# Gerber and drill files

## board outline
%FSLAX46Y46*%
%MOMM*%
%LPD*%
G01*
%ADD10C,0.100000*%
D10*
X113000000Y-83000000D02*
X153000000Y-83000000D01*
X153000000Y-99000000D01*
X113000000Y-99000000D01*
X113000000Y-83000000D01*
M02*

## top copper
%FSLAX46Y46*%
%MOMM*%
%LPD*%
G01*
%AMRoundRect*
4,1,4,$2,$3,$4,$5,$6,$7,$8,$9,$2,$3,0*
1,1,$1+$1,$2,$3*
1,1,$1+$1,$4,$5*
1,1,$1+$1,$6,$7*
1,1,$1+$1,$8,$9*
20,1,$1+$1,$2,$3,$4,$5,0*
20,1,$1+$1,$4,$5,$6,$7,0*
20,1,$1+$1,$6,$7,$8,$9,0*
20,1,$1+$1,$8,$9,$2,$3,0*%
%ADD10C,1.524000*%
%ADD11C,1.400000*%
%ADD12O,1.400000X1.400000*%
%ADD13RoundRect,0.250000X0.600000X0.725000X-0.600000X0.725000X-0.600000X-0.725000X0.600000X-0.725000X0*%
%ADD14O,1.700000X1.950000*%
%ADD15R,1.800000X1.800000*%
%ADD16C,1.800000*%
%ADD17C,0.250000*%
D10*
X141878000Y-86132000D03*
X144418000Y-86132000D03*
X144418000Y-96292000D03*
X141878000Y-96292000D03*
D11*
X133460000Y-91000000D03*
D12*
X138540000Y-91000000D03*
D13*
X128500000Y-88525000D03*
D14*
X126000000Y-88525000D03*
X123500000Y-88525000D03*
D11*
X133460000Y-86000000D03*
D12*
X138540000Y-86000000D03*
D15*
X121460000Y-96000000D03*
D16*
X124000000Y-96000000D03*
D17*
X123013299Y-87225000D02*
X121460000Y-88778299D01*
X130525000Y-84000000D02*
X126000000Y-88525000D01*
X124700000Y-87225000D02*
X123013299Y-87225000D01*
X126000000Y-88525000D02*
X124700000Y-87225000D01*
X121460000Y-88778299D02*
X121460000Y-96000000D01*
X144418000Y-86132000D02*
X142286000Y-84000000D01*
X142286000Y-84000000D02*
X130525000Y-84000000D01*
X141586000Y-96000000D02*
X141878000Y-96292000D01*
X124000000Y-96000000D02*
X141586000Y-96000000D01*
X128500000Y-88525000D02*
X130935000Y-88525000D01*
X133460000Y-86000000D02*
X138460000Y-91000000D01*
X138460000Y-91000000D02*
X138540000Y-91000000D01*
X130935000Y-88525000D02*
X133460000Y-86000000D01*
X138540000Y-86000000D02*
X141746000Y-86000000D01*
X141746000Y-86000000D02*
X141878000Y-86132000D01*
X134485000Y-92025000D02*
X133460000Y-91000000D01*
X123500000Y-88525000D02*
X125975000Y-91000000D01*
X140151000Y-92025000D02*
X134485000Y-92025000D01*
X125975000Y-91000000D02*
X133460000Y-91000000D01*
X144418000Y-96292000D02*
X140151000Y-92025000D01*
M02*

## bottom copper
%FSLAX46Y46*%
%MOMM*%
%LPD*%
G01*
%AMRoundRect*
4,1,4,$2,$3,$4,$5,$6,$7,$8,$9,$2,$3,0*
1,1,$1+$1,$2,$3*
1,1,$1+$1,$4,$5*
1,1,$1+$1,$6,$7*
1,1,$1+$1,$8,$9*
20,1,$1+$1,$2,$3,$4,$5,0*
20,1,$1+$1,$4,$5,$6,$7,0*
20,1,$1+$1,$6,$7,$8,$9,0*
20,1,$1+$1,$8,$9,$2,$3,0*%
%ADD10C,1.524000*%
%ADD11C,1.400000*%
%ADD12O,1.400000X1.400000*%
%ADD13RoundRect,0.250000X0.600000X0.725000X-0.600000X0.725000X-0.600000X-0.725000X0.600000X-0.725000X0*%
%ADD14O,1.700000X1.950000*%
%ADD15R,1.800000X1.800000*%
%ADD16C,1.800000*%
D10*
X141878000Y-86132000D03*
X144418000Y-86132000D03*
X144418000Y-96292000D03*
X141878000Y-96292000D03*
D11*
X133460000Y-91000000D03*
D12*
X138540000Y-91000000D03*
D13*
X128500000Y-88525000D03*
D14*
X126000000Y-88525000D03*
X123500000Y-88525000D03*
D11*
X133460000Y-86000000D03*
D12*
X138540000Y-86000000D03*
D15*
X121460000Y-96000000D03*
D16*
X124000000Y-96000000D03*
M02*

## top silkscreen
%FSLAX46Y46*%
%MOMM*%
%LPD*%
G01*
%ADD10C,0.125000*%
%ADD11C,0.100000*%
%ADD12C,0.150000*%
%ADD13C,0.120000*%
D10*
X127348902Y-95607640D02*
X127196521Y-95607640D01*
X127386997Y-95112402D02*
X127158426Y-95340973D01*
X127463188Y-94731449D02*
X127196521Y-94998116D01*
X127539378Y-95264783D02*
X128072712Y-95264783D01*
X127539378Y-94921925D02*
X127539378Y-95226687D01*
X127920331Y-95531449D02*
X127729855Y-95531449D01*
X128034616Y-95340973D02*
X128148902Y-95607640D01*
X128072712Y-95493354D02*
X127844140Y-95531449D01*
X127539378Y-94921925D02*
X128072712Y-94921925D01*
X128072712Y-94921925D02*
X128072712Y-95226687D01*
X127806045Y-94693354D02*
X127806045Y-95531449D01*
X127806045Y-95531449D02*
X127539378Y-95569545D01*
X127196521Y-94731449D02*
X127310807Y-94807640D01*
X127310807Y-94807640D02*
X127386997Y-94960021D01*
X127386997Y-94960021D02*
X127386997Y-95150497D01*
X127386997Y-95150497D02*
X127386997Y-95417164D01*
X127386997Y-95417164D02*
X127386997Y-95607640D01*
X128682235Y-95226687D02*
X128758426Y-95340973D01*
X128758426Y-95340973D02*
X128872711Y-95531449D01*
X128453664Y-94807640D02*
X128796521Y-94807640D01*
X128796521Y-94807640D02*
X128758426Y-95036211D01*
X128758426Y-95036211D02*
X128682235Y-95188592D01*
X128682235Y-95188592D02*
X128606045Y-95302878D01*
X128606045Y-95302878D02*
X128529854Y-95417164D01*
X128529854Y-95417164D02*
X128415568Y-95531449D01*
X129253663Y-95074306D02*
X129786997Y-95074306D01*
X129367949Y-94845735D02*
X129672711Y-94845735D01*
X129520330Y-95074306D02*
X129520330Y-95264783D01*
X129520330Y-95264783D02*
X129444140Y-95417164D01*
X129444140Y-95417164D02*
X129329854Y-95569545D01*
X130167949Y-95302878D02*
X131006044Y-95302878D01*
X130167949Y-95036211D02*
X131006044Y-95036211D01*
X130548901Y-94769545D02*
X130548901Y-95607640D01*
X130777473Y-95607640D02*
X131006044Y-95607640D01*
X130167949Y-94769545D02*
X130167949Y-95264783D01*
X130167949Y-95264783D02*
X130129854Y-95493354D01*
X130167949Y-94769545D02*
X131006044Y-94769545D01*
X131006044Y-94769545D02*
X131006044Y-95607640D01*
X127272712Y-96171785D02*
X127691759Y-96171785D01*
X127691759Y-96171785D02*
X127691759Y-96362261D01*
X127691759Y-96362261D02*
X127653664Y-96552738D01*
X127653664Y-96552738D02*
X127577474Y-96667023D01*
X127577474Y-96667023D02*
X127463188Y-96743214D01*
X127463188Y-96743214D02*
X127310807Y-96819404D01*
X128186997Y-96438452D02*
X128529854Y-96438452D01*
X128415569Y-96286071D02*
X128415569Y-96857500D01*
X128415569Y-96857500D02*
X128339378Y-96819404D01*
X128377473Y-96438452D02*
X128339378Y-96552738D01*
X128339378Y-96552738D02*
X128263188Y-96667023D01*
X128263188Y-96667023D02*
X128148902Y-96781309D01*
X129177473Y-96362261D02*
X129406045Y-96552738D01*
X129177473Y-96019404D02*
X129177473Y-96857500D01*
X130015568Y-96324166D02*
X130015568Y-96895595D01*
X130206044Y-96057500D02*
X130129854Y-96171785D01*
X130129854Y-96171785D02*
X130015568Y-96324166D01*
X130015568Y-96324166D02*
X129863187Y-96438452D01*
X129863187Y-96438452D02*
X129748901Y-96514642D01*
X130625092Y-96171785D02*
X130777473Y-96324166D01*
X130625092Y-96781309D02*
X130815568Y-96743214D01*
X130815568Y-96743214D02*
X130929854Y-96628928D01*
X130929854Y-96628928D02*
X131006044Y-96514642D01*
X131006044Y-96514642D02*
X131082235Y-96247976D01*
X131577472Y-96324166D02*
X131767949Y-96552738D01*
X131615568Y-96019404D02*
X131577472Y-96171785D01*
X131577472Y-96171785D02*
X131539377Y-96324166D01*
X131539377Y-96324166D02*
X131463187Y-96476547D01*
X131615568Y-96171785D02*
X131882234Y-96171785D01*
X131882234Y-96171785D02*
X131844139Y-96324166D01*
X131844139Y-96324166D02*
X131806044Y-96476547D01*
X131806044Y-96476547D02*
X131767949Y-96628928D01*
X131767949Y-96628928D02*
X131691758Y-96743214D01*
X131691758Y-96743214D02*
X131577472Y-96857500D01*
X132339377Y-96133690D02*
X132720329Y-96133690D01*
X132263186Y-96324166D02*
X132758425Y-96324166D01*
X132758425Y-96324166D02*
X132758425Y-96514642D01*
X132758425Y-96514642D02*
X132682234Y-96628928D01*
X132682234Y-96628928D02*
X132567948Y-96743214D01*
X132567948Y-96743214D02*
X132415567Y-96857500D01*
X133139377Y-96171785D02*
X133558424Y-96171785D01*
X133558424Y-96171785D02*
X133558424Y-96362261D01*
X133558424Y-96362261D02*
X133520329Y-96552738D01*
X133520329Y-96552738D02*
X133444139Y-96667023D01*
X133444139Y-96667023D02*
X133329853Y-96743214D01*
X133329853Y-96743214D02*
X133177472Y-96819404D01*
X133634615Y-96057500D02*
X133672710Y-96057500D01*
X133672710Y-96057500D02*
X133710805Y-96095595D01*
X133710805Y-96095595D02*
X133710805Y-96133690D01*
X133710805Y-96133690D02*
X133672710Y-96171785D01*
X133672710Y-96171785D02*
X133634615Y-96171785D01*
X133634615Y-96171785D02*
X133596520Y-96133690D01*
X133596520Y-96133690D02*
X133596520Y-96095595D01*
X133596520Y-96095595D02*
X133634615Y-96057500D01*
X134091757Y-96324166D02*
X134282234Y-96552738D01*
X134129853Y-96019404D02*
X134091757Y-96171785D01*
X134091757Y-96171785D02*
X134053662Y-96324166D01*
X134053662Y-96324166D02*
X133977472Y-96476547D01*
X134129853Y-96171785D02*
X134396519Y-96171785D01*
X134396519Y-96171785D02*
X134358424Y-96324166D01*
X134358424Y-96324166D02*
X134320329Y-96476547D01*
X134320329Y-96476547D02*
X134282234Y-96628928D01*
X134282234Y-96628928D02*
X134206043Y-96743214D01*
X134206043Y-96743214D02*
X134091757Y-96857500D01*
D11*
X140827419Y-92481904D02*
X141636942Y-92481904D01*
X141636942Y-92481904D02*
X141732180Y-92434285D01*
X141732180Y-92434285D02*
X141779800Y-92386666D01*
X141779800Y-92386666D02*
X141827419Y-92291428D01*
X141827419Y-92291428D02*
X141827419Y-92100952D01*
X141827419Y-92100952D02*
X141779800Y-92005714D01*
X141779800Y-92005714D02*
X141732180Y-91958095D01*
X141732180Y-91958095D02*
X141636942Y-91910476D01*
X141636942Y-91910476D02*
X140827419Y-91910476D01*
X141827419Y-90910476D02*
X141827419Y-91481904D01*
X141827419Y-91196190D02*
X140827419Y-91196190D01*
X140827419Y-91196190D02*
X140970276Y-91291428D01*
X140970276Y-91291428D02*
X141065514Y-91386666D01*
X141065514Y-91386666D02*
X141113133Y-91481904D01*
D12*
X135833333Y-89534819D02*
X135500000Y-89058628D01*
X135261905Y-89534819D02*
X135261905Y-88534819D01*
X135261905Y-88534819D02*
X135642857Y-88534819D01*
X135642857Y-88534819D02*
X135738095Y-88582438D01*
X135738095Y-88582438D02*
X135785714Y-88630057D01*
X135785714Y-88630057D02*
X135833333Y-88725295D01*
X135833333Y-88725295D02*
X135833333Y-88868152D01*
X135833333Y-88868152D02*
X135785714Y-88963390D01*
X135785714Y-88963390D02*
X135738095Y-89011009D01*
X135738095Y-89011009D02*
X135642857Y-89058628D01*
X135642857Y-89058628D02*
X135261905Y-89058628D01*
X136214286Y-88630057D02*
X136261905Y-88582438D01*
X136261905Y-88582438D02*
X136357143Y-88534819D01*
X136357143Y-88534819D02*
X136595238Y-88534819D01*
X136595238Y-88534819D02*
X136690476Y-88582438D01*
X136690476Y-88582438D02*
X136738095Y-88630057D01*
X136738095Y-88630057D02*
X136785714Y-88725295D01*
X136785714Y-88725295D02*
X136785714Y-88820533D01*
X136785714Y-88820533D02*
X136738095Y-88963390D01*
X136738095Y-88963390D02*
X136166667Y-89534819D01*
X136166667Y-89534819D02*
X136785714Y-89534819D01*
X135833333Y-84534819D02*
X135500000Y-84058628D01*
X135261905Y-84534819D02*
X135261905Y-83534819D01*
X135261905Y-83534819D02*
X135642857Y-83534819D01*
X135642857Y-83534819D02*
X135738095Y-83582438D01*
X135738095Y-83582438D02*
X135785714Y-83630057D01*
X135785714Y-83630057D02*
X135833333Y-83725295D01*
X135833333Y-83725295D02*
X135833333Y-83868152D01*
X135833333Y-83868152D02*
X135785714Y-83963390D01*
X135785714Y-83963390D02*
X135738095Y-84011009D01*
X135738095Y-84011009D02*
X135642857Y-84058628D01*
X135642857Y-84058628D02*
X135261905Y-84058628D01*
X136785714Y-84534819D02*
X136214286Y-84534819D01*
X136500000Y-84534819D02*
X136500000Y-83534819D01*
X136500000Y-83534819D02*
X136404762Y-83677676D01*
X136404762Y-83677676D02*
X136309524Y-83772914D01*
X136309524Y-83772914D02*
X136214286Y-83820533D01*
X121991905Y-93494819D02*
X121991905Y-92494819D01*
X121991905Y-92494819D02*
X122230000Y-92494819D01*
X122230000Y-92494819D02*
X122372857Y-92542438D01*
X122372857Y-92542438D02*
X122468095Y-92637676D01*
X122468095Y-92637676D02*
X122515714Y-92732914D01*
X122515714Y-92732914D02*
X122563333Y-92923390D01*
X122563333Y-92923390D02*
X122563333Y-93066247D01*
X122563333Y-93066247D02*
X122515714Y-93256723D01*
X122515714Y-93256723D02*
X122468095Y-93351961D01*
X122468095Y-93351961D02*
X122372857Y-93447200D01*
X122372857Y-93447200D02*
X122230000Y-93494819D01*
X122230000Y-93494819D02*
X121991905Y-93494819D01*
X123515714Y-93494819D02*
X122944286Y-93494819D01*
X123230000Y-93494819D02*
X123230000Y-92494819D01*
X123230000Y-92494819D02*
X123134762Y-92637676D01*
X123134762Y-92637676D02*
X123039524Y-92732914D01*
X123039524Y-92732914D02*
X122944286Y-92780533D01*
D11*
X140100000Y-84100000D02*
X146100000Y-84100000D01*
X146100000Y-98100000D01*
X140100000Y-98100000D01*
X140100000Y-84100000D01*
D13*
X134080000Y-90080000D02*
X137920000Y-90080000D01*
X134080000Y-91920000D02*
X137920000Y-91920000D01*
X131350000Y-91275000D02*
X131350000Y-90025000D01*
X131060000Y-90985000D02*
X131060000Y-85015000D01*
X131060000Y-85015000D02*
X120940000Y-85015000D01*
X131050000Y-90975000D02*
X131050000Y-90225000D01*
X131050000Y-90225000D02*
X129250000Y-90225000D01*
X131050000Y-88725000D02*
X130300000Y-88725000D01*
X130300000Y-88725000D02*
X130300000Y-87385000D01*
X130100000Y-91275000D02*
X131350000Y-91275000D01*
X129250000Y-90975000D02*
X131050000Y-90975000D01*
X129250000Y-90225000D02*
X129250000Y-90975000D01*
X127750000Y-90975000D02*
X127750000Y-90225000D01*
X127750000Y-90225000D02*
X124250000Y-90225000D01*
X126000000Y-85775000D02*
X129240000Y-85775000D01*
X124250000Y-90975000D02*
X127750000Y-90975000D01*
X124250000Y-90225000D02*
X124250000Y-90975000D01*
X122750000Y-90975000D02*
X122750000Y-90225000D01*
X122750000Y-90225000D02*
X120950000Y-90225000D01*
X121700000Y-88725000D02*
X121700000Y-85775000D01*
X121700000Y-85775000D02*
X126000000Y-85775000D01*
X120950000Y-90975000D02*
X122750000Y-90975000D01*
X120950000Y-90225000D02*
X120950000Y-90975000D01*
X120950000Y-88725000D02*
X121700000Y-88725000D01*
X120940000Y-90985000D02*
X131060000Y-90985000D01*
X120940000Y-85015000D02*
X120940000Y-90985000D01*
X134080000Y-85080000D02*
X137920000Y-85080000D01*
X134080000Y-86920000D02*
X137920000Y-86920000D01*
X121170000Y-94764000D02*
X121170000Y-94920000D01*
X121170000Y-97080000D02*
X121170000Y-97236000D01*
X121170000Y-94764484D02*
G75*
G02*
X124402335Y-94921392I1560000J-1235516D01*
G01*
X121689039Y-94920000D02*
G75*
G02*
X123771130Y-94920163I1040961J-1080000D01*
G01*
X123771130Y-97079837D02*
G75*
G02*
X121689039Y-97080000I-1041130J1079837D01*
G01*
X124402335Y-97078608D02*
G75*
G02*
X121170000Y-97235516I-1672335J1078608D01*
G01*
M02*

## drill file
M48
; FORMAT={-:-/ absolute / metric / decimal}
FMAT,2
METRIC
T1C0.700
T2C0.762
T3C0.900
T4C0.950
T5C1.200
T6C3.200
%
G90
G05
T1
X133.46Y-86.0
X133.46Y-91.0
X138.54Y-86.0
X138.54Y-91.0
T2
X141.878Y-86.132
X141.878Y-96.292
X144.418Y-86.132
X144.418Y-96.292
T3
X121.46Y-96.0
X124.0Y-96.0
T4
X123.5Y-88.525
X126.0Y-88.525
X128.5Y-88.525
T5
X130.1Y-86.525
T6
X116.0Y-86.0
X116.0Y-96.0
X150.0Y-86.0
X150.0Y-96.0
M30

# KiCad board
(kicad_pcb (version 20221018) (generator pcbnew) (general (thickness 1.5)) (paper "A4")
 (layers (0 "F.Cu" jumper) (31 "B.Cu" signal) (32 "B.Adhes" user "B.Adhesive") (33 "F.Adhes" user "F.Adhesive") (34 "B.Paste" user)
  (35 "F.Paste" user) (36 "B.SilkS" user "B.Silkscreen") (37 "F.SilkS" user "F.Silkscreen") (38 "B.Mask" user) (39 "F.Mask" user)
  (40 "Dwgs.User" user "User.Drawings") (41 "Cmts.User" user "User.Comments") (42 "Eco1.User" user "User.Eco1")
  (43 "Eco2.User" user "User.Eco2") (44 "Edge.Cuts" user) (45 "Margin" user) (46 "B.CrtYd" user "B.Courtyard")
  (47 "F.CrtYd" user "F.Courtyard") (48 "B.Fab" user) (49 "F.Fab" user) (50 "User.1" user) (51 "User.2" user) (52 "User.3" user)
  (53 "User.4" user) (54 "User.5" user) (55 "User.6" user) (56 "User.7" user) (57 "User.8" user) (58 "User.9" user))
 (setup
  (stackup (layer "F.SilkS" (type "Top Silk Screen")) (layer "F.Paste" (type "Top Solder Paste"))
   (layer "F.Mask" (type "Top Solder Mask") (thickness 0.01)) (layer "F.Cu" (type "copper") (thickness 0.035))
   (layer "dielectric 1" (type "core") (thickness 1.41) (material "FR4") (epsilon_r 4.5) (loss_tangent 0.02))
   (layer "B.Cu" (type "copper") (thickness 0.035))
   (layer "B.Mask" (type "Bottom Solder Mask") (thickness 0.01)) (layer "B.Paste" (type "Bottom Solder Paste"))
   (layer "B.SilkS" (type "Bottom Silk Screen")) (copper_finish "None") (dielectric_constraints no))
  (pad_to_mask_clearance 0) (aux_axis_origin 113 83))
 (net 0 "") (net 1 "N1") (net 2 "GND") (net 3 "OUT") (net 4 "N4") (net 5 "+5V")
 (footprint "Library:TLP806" (layer "F.Cu") (at 140.1 84.1)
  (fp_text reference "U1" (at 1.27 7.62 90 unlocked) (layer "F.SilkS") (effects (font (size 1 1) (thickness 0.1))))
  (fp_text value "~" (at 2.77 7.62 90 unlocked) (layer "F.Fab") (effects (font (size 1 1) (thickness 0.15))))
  (fp_rect (start 0 0) (end 6 14) (stroke (width 0.1) (type default)) (fill none) (layer "F.SilkS"))
  (pad "1" thru_hole circle (at 1.778 2.032) (size 1.524 1.524) (drill 0.762) (layers "*.Cu" "*.Mask") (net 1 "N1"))
  (pad "2" thru_hole circle (at 4.318 2.032) (size 1.524 1.524) (drill 0.762) (layers "*.Cu" "*.Mask") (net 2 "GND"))
  (pad "3" thru_hole circle (at 4.318 12.192) (size 1.524 1.524) (drill 0.762) (layers "*.Cu" "*.Mask") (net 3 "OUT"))
  (pad "4" thru_hole circle (at 1.778 12.192) (size 1.524 1.524) (drill 0.762) (layers "*.Cu" "*.Mask") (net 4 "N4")))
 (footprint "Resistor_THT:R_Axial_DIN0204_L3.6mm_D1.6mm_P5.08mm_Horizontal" (layer "F.Cu") (at 133.46 91)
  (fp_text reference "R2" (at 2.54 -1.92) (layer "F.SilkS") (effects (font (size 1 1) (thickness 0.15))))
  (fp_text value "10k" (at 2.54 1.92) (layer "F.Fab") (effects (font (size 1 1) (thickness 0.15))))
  (fp_line (start 0.62 -0.92) (end 4.46 -0.92) (stroke (width 0.12) (type solid)) (layer "F.SilkS"))
  (fp_line (start 0.62 0.92) (end 4.46 0.92) (stroke (width 0.12) (type solid)) (layer "F.SilkS"))
  (pad "1" thru_hole circle (at 0 0) (size 1.4 1.4) (drill 0.7) (layers "*.Cu" "*.Mask") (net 3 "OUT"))
  (pad "2" thru_hole oval (at 5.08 0) (size 1.4 1.4) (drill 0.7) (layers "*.Cu" "*.Mask") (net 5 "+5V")))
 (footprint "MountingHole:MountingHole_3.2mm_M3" (layer "F.Cu") (at 116 96)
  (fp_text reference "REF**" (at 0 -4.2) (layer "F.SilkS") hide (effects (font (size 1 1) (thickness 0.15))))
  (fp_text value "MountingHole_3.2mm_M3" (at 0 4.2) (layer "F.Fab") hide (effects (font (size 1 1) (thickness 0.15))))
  (pad "" np_thru_hole circle (at 0 0) (size 3.2 3.2) (drill 3.2) (layers "*.Cu" "*.Mask")))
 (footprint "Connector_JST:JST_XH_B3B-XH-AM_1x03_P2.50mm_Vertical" (layer "F.Cu") (at 128.5 88.525 180)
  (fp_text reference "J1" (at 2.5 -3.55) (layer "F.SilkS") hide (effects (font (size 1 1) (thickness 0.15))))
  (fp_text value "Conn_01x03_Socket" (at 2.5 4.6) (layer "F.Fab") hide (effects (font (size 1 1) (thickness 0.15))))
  (fp_line (start -2.85 -2.75) (end -2.85 -1.5) (stroke (width 0.12) (type solid)) (layer "F.SilkS"))
  (fp_line (start -2.56 -2.46) (end -2.56 3.51) (stroke (width 0.12) (type solid)) (layer "F.SilkS"))
  (fp_line (start -2.56 3.51) (end 7.56 3.51) (stroke (width 0.12) (type solid)) (layer "F.SilkS"))
  (fp_line (start -2.55 -2.45) (end -2.55 -1.7) (stroke (width 0.12) (type solid)) (layer "F.SilkS"))
  (fp_line (start -2.55 -1.7) (end -0.75 -1.7) (stroke (width 0.12) (type solid)) (layer "F.SilkS"))
  (fp_line (start -2.55 -0.2) (end -1.8 -0.2) (stroke (width 0.12) (type solid)) (layer "F.SilkS"))
  (fp_line (start -1.8 -0.2) (end -1.8 1.14) (stroke (width 0.12) (type solid)) (layer "F.SilkS"))
  (fp_line (start -1.6 -2.75) (end -2.85 -2.75) (stroke (width 0.12) (type solid)) (layer "F.SilkS"))
  (fp_line (start -0.75 -2.45) (end -2.55 -2.45) (stroke (width 0.12) (type solid)) (layer "F.SilkS"))
  (fp_line (start -0.75 -1.7) (end -0.75 -2.45) (stroke (width 0.12) (type solid)) (layer "F.SilkS"))
  (fp_line (start 0.75 -2.45) (end 0.75 -1.7) (stroke (width 0.12) (type solid)) (layer "F.SilkS"))
  (fp_line (start 0.75 -1.7) (end 4.25 -1.7) (stroke (width 0.12) (type solid)) (layer "F.SilkS"))
  (fp_line (start 2.5 2.75) (end -0.74 2.75) (stroke (width 0.12) (type solid)) (layer "F.SilkS"))
  (fp_line (start 4.25 -2.45) (end 0.75 -2.45) (stroke (width 0.12) (type solid)) (layer "F.SilkS"))
  (fp_line (start 4.25 -1.7) (end 4.25 -2.45) (stroke (width 0.12) (type solid)) (layer "F.SilkS"))
  (fp_line (start 5.75 -2.45) (end 5.75 -1.7) (stroke (width 0.12) (type solid)) (layer "F.SilkS"))
  (fp_line (start 5.75 -1.7) (end 7.55 -1.7) (stroke (width 0.12) (type solid)) (layer "F.SilkS"))
  (fp_line (start 6.8 -0.2) (end 6.8 2.75) (stroke (width 0.12) (type solid)) (layer "F.SilkS"))
  (fp_line (start 6.8 2.75) (end 2.5 2.75) (stroke (width 0.12) (type solid)) (layer "F.SilkS"))
  (fp_line (start 7.55 -2.45) (end 5.75 -2.45) (stroke (width 0.12) (type solid)) (layer "F.SilkS"))
  (fp_line (start 7.55 -1.7) (end 7.55 -2.45) (stroke (width 0.12) (type solid)) (layer "F.SilkS"))
  (fp_line (start 7.55 -0.2) (end 6.8 -0.2) (stroke (width 0.12) (type solid)) (layer "F.SilkS"))
  (fp_line (start 7.56 -2.46) (end -2.56 -2.46) (stroke (width 0.12) (type solid)) (layer "F.SilkS"))
  (fp_line (start 7.56 3.51) (end 7.56 -2.46) (stroke (width 0.12) (type solid)) (layer "F.SilkS"))
  (pad "" np_thru_hole circle (at -1.6 2 180) (size 1.2 1.2) (drill 1.2) (layers "*.Cu" "*.Mask"))
  (pad "1" thru_hole roundrect (at 0 0 180) (size 1.7 1.95) (drill 0.95) (layers "*.Cu" "*.Mask") (roundrect_rratio 0.1470588235)
   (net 5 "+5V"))
  (pad "2" thru_hole oval (at 2.5 0 180) (size 1.7 1.95) (drill 0.95) (layers "*.Cu" "*.Mask") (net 2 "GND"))
  (pad "3" thru_hole oval (at 5 0 180) (size 1.7 1.95) (drill 0.95) (layers "*.Cu" "*.Mask") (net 3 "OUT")))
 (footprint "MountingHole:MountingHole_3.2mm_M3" (layer "F.Cu") (at 150 86)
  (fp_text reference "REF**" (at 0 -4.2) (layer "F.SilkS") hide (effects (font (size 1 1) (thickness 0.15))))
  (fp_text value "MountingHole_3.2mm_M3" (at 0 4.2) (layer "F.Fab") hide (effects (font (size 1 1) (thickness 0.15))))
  (pad "" np_thru_hole circle (at 0 0) (size 3.2 3.2) (drill 3.2) (layers "*.Cu" "*.Mask")))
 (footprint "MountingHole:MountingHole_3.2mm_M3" (layer "F.Cu") (at 150 96)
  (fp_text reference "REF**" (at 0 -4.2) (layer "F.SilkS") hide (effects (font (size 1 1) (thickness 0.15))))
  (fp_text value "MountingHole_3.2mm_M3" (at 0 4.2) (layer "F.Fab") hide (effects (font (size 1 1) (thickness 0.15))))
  (pad "" np_thru_hole circle (at 0 0) (size 3.2 3.2) (drill 3.2) (layers "*.Cu" "*.Mask")))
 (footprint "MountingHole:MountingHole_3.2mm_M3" (layer "F.Cu") (at 116 86)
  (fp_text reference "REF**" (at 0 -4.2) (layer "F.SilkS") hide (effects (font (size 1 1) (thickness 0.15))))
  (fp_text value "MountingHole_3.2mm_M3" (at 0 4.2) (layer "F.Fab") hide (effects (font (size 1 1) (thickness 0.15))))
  (pad "" np_thru_hole circle (at 0 0) (size 3.2 3.2) (drill 3.2) (layers "F&B.Cu" "*.Mask")))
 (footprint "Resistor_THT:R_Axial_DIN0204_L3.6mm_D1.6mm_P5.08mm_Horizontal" (layer "F.Cu") (at 133.46 86)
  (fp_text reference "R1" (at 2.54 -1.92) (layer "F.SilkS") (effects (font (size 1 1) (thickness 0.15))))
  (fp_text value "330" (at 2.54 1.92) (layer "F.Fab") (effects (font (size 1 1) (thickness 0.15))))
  (fp_line (start 0.62 -0.92) (end 4.46 -0.92) (stroke (width 0.12) (type solid)) (layer "F.SilkS"))
  (fp_line (start 0.62 0.92) (end 4.46 0.92) (stroke (width 0.12) (type solid)) (layer "F.SilkS"))
  (pad "1" thru_hole circle (at 0 0) (size 1.4 1.4) (drill 0.7) (layers "*.Cu" "*.Mask") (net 5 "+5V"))
  (pad "2" thru_hole oval (at 5.08 0) (size 1.4 1.4) (drill 0.7) (layers "*.Cu" "*.Mask") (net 1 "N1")))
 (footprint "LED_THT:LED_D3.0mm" (layer "F.Cu") (at 121.46 96)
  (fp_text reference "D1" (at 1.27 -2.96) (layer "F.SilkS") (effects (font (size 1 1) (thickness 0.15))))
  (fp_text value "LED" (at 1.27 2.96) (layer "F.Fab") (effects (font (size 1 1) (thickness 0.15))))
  (fp_line (start -0.29 -1.236) (end -0.29 -1.08) (stroke (width 0.12) (type solid)) (layer "F.SilkS"))
  (fp_line (start -0.29 1.08) (end -0.29 1.236) (stroke (width 0.12) (type solid)) (layer "F.SilkS"))
  (fp_arc (start -0.29 -1.235516) (mid 1.366487 -1.987659) (end 2.942335 -1.078608) (stroke (width 0.12) (type solid)) (layer "F.SilkS"))
  (fp_arc (start 0.229039 -1.08) (mid 1.270117 -1.5) (end 2.31113 -1.079837) (stroke (width 0.12) (type solid)) (layer "F.SilkS"))
  (fp_arc (start 2.31113 1.079837) (mid 1.270117 1.5) (end 0.229039 1.08) (stroke (width 0.12) (type solid)) (layer "F.SilkS"))
  (fp_arc (start 2.942335 1.078608) (mid 1.366487 1.987659) (end -0.29 1.235516) (stroke (width 0.12) (type solid)) (layer "F.SilkS"))
  (pad "1" thru_hole rect (at 0 0) (size 1.8 1.8) (drill 0.9) (layers "*.Cu" "*.Mask") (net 2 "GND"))
  (pad "2" thru_hole circle (at 2.54 0) (size 1.8 1.8) (drill 0.9) (layers "*.Cu" "*.Mask") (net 4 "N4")))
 (gr_rect (start 113 83) (end 153 99) (stroke (width 0.1) (type default)) (fill none) (layer "Edge.Cuts"))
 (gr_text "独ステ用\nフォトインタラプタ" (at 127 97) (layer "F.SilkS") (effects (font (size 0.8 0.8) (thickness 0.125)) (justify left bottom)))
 (segment (start 123.013299 87.225) (end 121.46 88.778299) (width 0.25) (layer "F.Cu") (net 2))
 (segment (start 130.525 84) (end 126 88.525) (width 0.25) (layer "F.Cu") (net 2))
 (segment (start 124.7 87.225) (end 123.013299 87.225) (width 0.25) (layer "F.Cu") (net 2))
 (segment (start 126 88.525) (end 124.7 87.225) (width 0.25) (layer "F.Cu") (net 2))
 (segment (start 121.46 88.778299) (end 121.46 96) (width 0.25) (layer "F.Cu") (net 2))
 (segment (start 144.418 86.132) (end 142.286 84) (width 0.25) (layer "F.Cu") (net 2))
 (segment (start 142.286 84) (end 130.525 84) (width 0.25) (layer "F.Cu") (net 2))
 (segment (start 141.586 96) (end 141.878 96.292) (width 0.25) (layer "F.Cu") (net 4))
 (segment (start 124 96) (end 141.586 96) (width 0.25) (layer "F.Cu") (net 4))
 (segment (start 128.5 88.525) (end 130.935 88.525) (width 0.25) (layer "F.Cu") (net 5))
 (segment (start 133.46 86) (end 138.46 91) (width 0.25) (layer "F.Cu") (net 5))
 (segment (start 138.46 91) (end 138.54 91) (width 0.25) (layer "F.Cu") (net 5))
 (segment (start 130.935 88.525) (end 133.46 86) (width 0.25) (layer "F.Cu") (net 5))
 (segment (start 138.54 86) (end 141.746 86) (width 0.25) (layer "F.Cu") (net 1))
 (segment (start 141.746 86) (end 141.878 86.132) (width 0.25) (layer "F.Cu") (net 1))
 (segment (start 134.485 92.025) (end 133.46 91) (width 0.25) (layer "F.Cu") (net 3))
 (segment (start 123.5 88.525) (end 125.975 91) (width 0.25) (layer "F.Cu") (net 3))
 (segment (start 140.151 92.025) (end 134.485 92.025) (width 0.25) (layer "F.Cu") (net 3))
 (segment (start 125.975 91) (end 133.46 91) (width 0.25) (layer "F.Cu") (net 3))
 (segment (start 144.418 96.292) (end 140.151 92.025) (width 0.25) (layer "F.Cu") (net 3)))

